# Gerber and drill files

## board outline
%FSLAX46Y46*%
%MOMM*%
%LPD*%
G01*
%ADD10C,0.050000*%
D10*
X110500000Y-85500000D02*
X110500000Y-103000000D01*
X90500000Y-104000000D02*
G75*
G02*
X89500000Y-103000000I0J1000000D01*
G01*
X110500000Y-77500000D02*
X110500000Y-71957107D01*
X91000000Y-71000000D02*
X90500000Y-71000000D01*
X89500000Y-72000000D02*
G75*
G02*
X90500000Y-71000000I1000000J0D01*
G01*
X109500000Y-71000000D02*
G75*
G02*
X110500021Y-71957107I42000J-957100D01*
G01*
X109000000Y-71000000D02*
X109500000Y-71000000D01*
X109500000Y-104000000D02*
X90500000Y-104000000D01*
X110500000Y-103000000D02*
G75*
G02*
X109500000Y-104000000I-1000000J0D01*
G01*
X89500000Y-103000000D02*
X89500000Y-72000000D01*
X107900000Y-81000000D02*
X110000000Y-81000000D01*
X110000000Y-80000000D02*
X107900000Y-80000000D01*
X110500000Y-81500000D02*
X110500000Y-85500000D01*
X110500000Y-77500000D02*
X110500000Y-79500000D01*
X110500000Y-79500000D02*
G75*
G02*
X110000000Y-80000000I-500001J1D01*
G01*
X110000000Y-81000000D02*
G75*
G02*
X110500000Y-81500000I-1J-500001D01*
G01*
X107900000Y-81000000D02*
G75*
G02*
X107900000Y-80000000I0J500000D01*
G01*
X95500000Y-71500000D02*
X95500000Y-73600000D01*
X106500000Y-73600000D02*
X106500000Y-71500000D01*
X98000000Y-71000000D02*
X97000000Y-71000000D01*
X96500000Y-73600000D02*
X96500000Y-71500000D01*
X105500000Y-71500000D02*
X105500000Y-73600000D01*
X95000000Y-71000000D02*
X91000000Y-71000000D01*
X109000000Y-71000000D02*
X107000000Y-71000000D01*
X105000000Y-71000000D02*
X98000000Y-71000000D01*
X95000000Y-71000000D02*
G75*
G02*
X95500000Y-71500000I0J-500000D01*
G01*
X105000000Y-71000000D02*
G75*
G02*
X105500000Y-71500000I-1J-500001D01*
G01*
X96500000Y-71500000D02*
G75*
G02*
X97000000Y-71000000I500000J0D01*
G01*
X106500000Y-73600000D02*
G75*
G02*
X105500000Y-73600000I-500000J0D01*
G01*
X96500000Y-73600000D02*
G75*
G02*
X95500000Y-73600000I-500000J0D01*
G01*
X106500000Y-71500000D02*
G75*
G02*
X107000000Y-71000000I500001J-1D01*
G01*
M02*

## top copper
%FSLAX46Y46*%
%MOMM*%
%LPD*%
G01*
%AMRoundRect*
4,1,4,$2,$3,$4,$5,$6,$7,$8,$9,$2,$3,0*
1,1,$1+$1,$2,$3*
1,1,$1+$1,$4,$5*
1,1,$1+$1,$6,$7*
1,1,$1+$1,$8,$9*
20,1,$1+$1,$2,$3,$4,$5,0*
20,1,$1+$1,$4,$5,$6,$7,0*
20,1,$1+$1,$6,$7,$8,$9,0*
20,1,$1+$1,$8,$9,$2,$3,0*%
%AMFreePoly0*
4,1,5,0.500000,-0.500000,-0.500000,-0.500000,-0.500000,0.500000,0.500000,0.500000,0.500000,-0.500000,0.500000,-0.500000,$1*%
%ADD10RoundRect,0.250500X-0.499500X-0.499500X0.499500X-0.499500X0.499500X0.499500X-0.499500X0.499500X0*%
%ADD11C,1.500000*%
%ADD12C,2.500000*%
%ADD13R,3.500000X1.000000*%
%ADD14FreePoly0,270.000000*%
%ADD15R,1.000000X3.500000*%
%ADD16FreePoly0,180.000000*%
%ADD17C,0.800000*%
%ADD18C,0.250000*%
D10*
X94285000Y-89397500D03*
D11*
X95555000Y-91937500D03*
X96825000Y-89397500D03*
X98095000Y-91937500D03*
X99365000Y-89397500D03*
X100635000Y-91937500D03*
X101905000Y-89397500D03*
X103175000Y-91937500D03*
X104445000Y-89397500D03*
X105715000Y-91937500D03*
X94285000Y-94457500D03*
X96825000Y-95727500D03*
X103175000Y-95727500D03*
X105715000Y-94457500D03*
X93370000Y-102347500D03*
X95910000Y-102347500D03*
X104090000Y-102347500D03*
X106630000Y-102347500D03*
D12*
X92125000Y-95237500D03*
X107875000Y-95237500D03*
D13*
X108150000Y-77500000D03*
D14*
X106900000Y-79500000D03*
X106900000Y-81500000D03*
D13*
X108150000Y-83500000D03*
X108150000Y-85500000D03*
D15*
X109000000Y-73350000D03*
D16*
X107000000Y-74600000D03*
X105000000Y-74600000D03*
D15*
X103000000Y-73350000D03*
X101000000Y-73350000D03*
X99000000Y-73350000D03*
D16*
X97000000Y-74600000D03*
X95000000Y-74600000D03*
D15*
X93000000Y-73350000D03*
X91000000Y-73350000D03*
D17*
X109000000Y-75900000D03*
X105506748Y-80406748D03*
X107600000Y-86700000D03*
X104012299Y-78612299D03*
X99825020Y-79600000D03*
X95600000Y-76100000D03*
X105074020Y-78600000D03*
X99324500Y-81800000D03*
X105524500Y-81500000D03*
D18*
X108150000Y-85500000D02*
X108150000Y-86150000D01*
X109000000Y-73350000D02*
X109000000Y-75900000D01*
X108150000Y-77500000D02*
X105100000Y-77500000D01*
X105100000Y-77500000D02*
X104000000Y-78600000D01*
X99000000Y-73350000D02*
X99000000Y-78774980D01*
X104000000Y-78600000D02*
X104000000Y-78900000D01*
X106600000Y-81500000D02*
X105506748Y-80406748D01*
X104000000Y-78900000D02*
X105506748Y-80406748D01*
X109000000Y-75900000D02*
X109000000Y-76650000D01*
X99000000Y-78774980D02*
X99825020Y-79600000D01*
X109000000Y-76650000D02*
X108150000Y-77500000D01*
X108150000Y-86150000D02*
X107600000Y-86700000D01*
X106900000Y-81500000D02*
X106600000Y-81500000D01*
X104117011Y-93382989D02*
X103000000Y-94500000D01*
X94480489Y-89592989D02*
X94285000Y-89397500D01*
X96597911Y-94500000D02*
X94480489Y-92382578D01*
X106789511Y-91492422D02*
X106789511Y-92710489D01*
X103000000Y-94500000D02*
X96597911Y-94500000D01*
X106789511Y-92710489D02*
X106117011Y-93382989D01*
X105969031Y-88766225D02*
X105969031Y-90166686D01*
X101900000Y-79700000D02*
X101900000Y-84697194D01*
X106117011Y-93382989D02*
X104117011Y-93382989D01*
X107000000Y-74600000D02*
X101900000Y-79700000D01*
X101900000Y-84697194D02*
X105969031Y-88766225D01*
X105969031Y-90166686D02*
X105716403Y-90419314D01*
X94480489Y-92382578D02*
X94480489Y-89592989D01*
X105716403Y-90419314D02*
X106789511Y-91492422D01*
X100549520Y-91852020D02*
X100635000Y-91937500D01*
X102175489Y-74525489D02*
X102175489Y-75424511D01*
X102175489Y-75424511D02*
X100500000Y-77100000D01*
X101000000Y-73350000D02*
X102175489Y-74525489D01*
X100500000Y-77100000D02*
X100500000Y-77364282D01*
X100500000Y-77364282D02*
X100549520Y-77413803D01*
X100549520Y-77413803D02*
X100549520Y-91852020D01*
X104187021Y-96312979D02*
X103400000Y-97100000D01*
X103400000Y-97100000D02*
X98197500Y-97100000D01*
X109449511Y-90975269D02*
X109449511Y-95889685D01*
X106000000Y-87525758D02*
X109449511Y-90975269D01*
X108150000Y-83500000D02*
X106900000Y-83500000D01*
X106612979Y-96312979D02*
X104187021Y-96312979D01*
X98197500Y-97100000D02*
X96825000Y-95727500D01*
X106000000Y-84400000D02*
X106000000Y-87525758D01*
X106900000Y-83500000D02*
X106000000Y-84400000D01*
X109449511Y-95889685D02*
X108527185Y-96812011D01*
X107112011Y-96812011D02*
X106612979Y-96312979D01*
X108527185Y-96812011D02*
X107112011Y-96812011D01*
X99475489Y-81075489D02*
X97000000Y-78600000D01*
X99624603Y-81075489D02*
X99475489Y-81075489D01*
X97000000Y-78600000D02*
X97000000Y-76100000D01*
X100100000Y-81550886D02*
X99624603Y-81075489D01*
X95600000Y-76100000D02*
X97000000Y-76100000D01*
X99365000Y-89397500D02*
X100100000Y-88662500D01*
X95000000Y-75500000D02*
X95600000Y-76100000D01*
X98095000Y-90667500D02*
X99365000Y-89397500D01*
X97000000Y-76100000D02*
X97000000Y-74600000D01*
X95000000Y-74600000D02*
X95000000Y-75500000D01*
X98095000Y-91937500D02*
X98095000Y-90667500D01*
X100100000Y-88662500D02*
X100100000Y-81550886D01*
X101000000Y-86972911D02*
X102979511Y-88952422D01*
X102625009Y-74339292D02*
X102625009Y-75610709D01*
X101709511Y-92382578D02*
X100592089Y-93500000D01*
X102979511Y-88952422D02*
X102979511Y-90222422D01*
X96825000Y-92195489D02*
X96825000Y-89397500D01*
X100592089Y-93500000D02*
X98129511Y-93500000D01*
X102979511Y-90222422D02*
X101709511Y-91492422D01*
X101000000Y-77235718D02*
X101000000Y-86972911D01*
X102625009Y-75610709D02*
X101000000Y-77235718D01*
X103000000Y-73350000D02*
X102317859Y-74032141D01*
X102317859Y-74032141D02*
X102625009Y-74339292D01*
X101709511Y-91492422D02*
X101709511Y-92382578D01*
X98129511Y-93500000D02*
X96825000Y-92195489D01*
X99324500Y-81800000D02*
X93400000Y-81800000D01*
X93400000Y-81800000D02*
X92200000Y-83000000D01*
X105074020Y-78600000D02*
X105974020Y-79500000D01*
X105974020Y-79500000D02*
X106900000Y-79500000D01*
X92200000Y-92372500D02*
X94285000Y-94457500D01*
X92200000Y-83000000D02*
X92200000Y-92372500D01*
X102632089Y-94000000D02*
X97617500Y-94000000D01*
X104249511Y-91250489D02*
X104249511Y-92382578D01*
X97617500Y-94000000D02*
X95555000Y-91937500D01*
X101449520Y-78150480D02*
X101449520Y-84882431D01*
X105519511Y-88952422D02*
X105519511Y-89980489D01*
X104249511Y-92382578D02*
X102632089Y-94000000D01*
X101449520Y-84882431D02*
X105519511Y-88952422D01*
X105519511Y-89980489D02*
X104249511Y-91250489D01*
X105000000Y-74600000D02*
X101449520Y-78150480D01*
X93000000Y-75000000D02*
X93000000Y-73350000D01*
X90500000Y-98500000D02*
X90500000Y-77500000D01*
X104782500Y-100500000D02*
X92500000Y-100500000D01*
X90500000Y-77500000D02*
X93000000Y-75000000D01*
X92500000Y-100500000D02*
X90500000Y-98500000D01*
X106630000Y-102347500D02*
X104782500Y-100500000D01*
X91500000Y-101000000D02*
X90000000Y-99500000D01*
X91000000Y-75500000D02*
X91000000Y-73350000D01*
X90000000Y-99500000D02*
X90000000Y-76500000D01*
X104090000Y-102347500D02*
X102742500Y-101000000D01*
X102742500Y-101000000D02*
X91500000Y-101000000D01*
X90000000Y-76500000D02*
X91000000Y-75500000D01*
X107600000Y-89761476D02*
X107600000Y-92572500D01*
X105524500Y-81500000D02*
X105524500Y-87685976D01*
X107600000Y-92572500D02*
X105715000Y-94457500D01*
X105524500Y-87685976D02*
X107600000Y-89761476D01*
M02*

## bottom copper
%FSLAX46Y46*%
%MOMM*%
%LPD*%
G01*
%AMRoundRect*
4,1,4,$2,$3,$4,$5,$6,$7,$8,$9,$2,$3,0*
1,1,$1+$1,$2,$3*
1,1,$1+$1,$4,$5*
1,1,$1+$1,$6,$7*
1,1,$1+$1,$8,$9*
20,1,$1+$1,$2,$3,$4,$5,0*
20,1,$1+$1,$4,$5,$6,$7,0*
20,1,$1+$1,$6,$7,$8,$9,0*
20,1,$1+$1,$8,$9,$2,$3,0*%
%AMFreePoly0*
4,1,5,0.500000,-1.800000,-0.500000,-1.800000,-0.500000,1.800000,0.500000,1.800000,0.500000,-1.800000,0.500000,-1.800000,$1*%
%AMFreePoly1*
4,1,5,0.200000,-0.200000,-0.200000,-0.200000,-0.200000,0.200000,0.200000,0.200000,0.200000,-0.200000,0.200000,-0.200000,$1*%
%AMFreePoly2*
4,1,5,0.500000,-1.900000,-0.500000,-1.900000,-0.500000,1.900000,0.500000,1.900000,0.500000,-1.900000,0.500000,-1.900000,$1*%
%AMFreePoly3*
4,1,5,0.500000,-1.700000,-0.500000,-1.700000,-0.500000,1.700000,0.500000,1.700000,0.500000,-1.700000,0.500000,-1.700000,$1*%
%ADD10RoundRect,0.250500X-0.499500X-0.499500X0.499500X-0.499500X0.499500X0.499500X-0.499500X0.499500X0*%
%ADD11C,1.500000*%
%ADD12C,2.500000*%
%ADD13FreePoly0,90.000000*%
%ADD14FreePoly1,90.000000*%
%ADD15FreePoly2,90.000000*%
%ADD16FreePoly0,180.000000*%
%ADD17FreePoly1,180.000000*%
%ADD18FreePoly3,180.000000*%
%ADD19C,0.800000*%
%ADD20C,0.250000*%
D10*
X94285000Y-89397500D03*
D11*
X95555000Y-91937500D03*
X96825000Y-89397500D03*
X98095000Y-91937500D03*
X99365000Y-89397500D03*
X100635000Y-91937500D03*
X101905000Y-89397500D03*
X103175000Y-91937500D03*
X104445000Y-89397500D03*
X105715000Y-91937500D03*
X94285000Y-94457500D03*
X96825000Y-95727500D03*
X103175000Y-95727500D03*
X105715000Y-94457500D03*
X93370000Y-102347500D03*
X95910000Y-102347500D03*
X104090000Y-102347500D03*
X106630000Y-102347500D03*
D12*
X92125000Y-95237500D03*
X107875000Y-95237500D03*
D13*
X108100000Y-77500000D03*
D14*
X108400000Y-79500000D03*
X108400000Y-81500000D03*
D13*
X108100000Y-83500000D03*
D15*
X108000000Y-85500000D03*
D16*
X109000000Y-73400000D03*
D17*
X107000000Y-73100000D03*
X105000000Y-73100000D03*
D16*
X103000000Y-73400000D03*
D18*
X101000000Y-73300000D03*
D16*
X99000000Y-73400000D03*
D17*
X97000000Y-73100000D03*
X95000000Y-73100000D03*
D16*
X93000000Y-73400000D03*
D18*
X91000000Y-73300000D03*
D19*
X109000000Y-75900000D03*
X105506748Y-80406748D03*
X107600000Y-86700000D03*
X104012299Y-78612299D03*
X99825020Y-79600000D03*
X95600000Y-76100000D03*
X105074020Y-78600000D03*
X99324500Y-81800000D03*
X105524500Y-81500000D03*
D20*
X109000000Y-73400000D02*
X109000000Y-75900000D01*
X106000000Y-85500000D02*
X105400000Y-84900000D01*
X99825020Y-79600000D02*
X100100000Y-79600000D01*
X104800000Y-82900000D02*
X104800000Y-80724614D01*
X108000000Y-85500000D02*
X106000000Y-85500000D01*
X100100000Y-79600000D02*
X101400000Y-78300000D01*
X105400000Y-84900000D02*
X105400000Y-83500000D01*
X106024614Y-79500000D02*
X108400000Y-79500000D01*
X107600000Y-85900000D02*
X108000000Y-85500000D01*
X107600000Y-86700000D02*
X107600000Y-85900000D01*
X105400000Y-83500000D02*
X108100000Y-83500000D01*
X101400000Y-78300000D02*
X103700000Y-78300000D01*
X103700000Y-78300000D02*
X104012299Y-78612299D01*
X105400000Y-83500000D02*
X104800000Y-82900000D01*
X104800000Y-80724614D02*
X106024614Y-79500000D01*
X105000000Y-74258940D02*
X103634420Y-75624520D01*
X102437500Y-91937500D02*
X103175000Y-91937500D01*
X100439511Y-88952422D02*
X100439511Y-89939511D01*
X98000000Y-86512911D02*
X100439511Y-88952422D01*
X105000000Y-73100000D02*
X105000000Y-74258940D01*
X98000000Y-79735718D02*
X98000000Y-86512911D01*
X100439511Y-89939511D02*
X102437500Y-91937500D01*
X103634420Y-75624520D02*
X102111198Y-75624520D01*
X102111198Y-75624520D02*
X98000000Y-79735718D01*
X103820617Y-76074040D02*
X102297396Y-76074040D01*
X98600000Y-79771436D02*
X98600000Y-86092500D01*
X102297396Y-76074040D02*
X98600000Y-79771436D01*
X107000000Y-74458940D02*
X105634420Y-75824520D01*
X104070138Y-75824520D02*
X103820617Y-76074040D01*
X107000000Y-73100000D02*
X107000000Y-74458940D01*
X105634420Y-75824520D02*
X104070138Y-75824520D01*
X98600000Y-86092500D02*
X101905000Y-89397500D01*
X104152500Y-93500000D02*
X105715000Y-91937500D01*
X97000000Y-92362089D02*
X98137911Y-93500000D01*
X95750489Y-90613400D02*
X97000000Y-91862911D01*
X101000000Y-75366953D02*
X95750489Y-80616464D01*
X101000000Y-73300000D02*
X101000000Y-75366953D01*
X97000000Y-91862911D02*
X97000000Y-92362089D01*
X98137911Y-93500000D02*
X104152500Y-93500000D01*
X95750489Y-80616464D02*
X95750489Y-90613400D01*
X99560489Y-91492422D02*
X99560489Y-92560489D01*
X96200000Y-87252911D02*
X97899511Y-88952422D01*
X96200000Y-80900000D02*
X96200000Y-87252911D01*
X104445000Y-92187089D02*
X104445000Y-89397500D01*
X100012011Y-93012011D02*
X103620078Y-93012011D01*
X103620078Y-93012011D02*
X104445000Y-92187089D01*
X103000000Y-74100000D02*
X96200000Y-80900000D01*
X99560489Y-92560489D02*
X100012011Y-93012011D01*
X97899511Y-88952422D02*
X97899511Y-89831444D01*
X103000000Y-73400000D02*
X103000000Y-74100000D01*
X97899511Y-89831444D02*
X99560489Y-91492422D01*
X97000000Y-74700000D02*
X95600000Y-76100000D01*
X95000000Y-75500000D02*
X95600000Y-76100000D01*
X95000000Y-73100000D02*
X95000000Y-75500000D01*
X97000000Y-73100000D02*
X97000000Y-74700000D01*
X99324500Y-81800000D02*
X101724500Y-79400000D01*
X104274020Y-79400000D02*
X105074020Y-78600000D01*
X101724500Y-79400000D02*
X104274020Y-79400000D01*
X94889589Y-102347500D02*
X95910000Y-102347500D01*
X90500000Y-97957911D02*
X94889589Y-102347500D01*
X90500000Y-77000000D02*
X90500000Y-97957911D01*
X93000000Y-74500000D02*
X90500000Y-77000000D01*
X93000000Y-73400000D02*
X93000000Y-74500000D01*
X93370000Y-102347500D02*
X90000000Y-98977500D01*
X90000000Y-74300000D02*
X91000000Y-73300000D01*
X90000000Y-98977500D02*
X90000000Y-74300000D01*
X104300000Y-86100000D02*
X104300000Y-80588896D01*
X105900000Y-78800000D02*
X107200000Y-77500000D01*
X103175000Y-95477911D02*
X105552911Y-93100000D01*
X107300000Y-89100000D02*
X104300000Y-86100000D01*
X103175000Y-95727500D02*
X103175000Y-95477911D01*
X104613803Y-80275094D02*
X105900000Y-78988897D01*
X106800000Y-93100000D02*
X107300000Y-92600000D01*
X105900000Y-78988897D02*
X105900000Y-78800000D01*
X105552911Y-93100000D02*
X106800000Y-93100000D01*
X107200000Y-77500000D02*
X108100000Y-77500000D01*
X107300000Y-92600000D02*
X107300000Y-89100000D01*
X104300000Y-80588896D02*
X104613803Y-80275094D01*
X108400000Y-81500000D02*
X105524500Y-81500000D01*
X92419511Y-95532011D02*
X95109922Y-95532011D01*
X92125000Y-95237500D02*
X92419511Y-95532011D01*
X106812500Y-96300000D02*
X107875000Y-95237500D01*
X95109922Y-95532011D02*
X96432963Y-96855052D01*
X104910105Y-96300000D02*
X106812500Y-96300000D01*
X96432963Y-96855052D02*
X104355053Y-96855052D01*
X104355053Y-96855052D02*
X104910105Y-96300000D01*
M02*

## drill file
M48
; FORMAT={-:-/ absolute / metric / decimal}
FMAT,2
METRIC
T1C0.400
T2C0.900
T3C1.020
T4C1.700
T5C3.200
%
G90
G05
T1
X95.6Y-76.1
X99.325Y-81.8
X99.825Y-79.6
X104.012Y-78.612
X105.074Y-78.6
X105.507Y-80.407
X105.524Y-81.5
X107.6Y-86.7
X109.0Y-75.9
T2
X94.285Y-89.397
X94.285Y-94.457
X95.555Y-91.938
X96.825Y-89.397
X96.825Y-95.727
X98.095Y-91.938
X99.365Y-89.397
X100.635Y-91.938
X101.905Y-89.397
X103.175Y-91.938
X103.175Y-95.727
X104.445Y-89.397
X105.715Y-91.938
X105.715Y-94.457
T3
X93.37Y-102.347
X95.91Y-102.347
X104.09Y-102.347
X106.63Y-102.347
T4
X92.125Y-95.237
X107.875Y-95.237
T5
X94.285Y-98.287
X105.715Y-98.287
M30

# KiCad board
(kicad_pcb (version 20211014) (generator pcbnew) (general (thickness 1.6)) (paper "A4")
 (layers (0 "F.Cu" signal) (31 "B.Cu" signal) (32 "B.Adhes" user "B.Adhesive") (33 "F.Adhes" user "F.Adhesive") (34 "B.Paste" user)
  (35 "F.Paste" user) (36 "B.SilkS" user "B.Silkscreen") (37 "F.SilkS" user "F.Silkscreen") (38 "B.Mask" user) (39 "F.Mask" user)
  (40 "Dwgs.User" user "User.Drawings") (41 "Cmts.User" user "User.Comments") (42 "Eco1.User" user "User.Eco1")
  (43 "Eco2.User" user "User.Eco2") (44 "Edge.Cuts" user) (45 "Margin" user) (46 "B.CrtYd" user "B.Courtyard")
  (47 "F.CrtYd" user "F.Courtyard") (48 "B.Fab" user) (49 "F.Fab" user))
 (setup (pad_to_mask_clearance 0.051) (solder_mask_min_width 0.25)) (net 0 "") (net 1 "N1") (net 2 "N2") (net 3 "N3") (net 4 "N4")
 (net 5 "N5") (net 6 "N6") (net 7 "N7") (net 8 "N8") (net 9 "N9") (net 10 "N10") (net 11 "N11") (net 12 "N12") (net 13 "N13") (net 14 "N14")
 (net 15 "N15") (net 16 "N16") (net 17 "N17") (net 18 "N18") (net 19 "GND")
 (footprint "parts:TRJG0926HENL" (layer "F.Cu") (at 100 98.2875)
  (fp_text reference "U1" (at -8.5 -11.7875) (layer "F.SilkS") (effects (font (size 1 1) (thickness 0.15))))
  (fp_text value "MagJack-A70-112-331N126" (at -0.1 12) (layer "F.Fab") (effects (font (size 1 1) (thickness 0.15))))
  (pad "" np_thru_hole circle locked (at -5.715 0) (size 3.2 3.2) (drill 3.2) (layers *.Cu *.Mask))
  (pad "" np_thru_hole circle locked (at 5.715 0) (size 3.2 3.2) (drill 3.2) (layers *.Cu *.Mask))
  (pad "1" thru_hole roundrect locked (at -5.715 -8.89) (size 1.5 1.5) (drill 0.9) (layers *.Cu *.Mask) (roundrect_rratio 0.167)
   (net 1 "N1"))
  (pad "2" thru_hole circle locked (at -4.445 -6.35) (size 1.5 1.5) (drill 0.9) (layers *.Cu *.Mask) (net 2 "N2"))
  (pad "3" thru_hole circle locked (at -3.175 -8.89) (size 1.5 1.5) (drill 0.9) (layers *.Cu *.Mask) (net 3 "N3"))
  (pad "4" thru_hole circle locked (at -1.905 -6.35) (size 1.5 1.5) (drill 0.9) (layers *.Cu *.Mask) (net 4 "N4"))
  (pad "5" thru_hole circle locked (at -0.635 -8.89) (size 1.5 1.5) (drill 0.9) (layers *.Cu *.Mask) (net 4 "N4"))
  (pad "6" thru_hole circle locked (at 0.635 -6.35 90) (size 1.5 1.5) (drill 0.9) (layers *.Cu *.Mask) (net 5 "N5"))
  (pad "7" thru_hole circle locked (at 1.905 -8.89) (size 1.5 1.5) (drill 0.9) (layers *.Cu *.Mask) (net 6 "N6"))
  (pad "8" thru_hole circle locked (at 3.175 -6.35) (size 1.5 1.5) (drill 0.9) (layers *.Cu *.Mask) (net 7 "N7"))
  (pad "9" thru_hole circle locked (at 4.445 -8.89) (size 1.5 1.5) (drill 0.9) (layers *.Cu *.Mask) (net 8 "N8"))
  (pad "10" thru_hole circle locked (at 5.715 -6.35) (size 1.5 1.5) (drill 0.9) (layers *.Cu *.Mask) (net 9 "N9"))
  (pad "11" thru_hole circle locked (at -5.715 -3.83) (size 1.5 1.5) (drill 0.9) (layers *.Cu *.Mask) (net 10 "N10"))
  (pad "12" thru_hole circle locked (at -3.175 -2.56) (size 1.5 1.5) (drill 0.9) (layers *.Cu *.Mask) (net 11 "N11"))
  (pad "13" thru_hole circle locked (at 3.175 -2.56) (size 1.5 1.5) (drill 0.9) (layers *.Cu *.Mask) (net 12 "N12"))
  (pad "14" thru_hole circle locked (at 5.715 -3.83) (size 1.5 1.5) (drill 0.9) (layers *.Cu *.Mask) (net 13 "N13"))
  (pad "15" thru_hole circle locked (at -6.63 4.06) (size 1.5 1.5) (drill 1.02) (layers *.Cu *.Mask) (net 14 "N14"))
  (pad "16" thru_hole circle locked (at -4.09 4.06) (size 1.5 1.5) (drill 1.02) (layers *.Cu *.Mask) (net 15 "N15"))
  (pad "17" thru_hole circle locked (at 4.09 4.06) (size 1.5 1.5) (drill 1.02) (layers *.Cu *.Mask) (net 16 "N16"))
  (pad "18" thru_hole circle locked (at 6.63 4.06) (size 1.5 1.5) (drill 1.02) (layers *.Cu *.Mask) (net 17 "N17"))
  (pad "19" thru_hole circle locked (at -7.875 -3.05) (size 2.5 2.5) (drill 1.7) (layers *.Cu *.Mask) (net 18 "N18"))
  (pad "20" thru_hole circle locked (at 7.875 -3.05) (size 2.5 2.5) (drill 1.7) (layers *.Cu *.Mask) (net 18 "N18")))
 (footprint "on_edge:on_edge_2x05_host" (layer "F.Cu") (at 110.5 81.5 -90)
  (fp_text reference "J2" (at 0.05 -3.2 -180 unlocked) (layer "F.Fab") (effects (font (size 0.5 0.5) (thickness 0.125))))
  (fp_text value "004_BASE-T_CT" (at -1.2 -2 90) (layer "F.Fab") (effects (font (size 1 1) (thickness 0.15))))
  (fp_line (start -0.5 2.6) (end -0.5 0.5) (layer "Edge.Cuts") (width 0.05))
  (fp_line (start -1.5 0.5) (end -1.5 2.6) (layer "Edge.Cuts") (width 0.05))
  (fp_line (start 0 0) (end 4 0) (layer "Edge.Cuts") (width 0.05))
  (fp_line (start -4 0) (end -2 0) (layer "Edge.Cuts") (width 0.05))
  (fp_arc (start -2 0) (mid -1.646447 0.146447) (end -1.5 0.5) (layer "Edge.Cuts") (width 0.05))
  (fp_arc (start -0.5 0.5) (mid -0.353553 0.146447) (end 0 0) (layer "Edge.Cuts") (width 0.05))
  (fp_arc (start -0.5 2.6) (mid -1 3.1) (end -1.5 2.6) (layer "Edge.Cuts") (width 0.05))
  (pad "1" smd rect locked (at -4 2.35 270) (size 1 3.5) (layers "F.Cu" "F.Mask") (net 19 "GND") (zone_connect 0))
  (pad "2" smd custom locked (at -2 3.6 270) (size 1 1) (layers "F.Cu" "F.Mask") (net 10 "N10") (zone_connect 0)
   (options (clearance outline) (anchor rect)) (primitives))
  (pad "3" smd custom locked (at 0 3.6 270) (size 1 1) (layers "F.Cu" "F.Mask") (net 19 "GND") (zone_connect 0)
   (options (clearance outline) (anchor rect)) (primitives))
  (pad "4" smd rect locked (at 2 2.35 270) (size 1 3.5) (layers "F.Cu" "F.Mask") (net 11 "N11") (zone_connect 0))
  (pad "5" smd rect locked (at 4 2.35 270) (size 1 3.5) (layers "F.Cu" "F.Mask") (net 19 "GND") (zone_connect 0))
  (pad "6" smd custom locked (at -4 2.4 90) (size 1 3.6) (layers "B.Cu" "B.Mask") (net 12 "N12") (zone_connect 0)
   (options (clearance outline) (anchor rect)) (primitives))
  (pad "7" smd custom locked (at -2 2.1 90) (size 0.4 0.4) (layers "B.Cu" "B.Mask") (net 19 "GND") (zone_connect 0)
   (options (clearance outline) (anchor rect)) (primitives))
  (pad "8" smd custom locked (at 0 2.1 90) (size 0.4 0.4) (layers "B.Cu" "B.Mask") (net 13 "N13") (zone_connect 0)
   (options (clearance outline) (anchor rect)) (primitives))
  (pad "9" smd custom locked (at 2 2.4 90) (size 1 3.6) (layers "B.Cu" "B.Mask") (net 19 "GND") (zone_connect 0)
   (options (clearance outline) (anchor rect)) (primitives))
  (pad "10" smd custom locked (at 4 2.5 90) (size 1 3.8) (layers "B.Cu" "B.Mask") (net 19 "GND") (zone_connect 0)
   (options (clearance outline) (anchor rect)) (primitives)))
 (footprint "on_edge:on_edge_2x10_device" (layer "F.Cu") (at 105 71 180)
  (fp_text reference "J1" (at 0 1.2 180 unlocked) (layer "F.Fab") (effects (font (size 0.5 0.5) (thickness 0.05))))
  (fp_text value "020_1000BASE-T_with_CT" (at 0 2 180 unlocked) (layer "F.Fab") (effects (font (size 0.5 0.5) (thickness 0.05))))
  (fp_line (start 9.5 -0.5) (end 9.5 -2.6) (layer "Edge.Cuts") (width 0.05))
  (fp_line (start -1.5 -2.6) (end -1.5 -0.5) (layer "Edge.Cuts") (width 0.05))
  (fp_line (start 7 0) (end 8 0) (layer "Edge.Cuts") (width 0.05))
  (fp_line (start 8.5 -2.6) (end 8.5 -0.5) (layer "Edge.Cuts") (width 0.05))
  (fp_line (start -0.5 -0.5) (end -0.5 -2.6) (layer "Edge.Cuts") (width 0.05))
  (fp_line (start 10 0) (end 14 0) (layer "Edge.Cuts") (width 0.05))
  (fp_line (start -4 0) (end -2 0) (layer "Edge.Cuts") (width 0.05))
  (fp_line (start 0 0) (end 7 0) (layer "Edge.Cuts") (width 0.05))
  (fp_arc (start 10 0) (mid 9.646447 -0.146447) (end 9.5 -0.5) (layer "Edge.Cuts") (width 0.05))
  (fp_arc (start 0 0) (mid -0.353553 -0.146447) (end -0.5 -0.5) (layer "Edge.Cuts") (width 0.05))
  (fp_arc (start 8.5 -0.5) (mid 8.353553 -0.146447) (end 8 0) (layer "Edge.Cuts") (width 0.05))
  (fp_arc (start -1.5 -2.6) (mid -1 -3.1) (end -0.5 -2.6) (layer "Edge.Cuts") (width 0.05))
  (fp_arc (start 8.5 -2.6) (mid 9 -3.1) (end 9.5 -2.6) (layer "Edge.Cuts") (width 0.05))
  (fp_arc (start -1.5 -0.5) (mid -1.646447 -0.146447) (end -2 0) (layer "Edge.Cuts") (width 0.05))
  (pad "1" smd rect locked (at -4 -2.35) (size 1 3.5) (layers "F.Cu" "F.Mask") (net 19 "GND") (zone_connect 0))
  (pad "2" smd custom locked (at -2 -3.6 180) (size 1 1) (layers "F.Cu" "F.Mask") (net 1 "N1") (zone_connect 0)
   (options (clearance outline) (anchor rect)) (primitives))
  (pad "3" smd custom locked (at 0 -3.6 180) (size 1 1) (layers "F.Cu" "F.Mask") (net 2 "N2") (zone_connect 0)
   (options (clearance outline) (anchor rect)) (primitives))
  (pad "4" smd rect locked (at 2 -2.35) (size 1 3.5) (layers "F.Cu" "F.Mask") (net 3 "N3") (zone_connect 0))
  (pad "5" smd rect locked (at 4 -2.35) (size 1 3.5) (layers "F.Cu" "F.Mask") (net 5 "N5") (zone_connect 0))
  (pad "6" smd rect locked (at 6 -2.35) (size 1 3.5) (layers "F.Cu" "F.Mask") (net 19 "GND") (zone_connect 0))
  (pad "7" smd custom locked (at 8 -3.6 180) (size 1 1) (layers "F.Cu" "F.Mask") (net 4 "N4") (zone_connect 0)
   (options (clearance outline) (anchor rect)) (primitives))
  (pad "8" smd custom locked (at 10 -3.6 180) (size 1 1) (layers "F.Cu" "F.Mask") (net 4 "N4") (zone_connect 0)
   (options (clearance outline) (anchor rect)) (primitives))
  (pad "9" smd rect locked (at 12 -2.35) (size 1 3.5) (layers "F.Cu" "F.Mask") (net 17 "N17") (zone_connect 0))
  (pad "10" smd rect locked (at 14 -2.35) (size 1 3.5) (layers "F.Cu" "F.Mask") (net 16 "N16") (zone_connect 0))
  (pad "11" smd custom locked (at -4 -2.4 180) (size 1 3.6) (layers "B.Cu" "B.Mask") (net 19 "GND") (zone_connect 0)
   (options (clearance outline) (anchor rect)) (primitives))
  (pad "12" smd custom locked (at -2 -2.1 180) (size 0.4 0.4) (layers "B.Cu" "B.Mask") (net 6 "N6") (zone_connect 0)
   (options (clearance outline) (anchor rect)) (primitives))
  (pad "13" smd custom locked (at 0 -2.1 180) (size 0.4 0.4) (layers "B.Cu" "B.Mask") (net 7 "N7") (zone_connect 0)
   (options (clearance outline) (anchor rect)) (primitives))
  (pad "14" smd custom locked (at 2 -2.4 180) (size 1 3.6) (layers "B.Cu" "B.Mask") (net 8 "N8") (zone_connect 0)
   (options (clearance outline) (anchor rect)) (primitives))
  (pad "15" smd custom locked (at 4 -2.3 180) (size 1 3.4) (layers "B.Cu" "B.Mask") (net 9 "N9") (zone_connect 0)
   (options (clearance outline) (anchor rect)) (primitives))
  (pad "16" smd custom locked (at 6 -2.4 180) (size 1 3.6) (layers "B.Cu" "B.Mask") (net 19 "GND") (zone_connect 0)
   (options (clearance outline) (anchor rect)) (primitives))
  (pad "17" smd custom locked (at 8 -2.1 180) (size 0.4 0.4) (layers "B.Cu" "B.Mask") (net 4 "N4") (zone_connect 0)
   (options (clearance outline) (anchor rect)) (primitives))
  (pad "18" smd custom locked (at 10 -2.1 180) (size 0.4 0.4) (layers "B.Cu" "B.Mask") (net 4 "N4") (zone_connect 0)
   (options (clearance outline) (anchor rect)) (primitives))
  (pad "19" smd custom locked (at 12 -2.4 180) (size 1 3.6) (layers "B.Cu" "B.Mask") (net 15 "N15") (zone_connect 0)
   (options (clearance outline) (anchor rect)) (primitives))
  (pad "20" smd custom locked (at 14 -2.3 180) (size 1 3.4) (layers "B.Cu" "B.Mask") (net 14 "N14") (zone_connect 0)
   (options (clearance outline) (anchor rect)) (primitives)))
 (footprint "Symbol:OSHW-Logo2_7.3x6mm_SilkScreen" (layer "B.Cu") (at 99 82 180)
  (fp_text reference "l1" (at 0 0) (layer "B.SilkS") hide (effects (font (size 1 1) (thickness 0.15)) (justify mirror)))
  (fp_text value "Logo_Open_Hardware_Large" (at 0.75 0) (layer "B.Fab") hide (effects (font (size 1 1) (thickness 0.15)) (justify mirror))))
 (gr_line (start 110.5 85.5) (end 110.5 103) (layer "Edge.Cuts") (width 0.05))
 (gr_arc (start 90.5 104) (mid 89.792893 103.707107) (end 89.5 103) (layer "Edge.Cuts") (width 0.05))
 (gr_line (start 110.5 77.5) (end 110.5 71.957107) (layer "Edge.Cuts") (width 0.05))
 (gr_line (start 91 71) (end 90.5 71) (layer "Edge.Cuts") (width 0.05))
 (gr_arc (start 89.5 72) (mid 89.792893 71.292893) (end 90.5 71) (layer "Edge.Cuts") (width 0.05))
 (gr_arc (start 109.5 71) (mid 110.204395 71.264999) (end 110.5 71.957107) (layer "Edge.Cuts") (width 0.05))
 (gr_line (start 109 71) (end 109.5 71) (layer "Edge.Cuts") (width 0.05))
 (gr_line (start 109.5 104) (end 90.5 104) (layer "Edge.Cuts") (width 0.05))
 (gr_arc (start 110.5 103) (mid 110.207107 103.707107) (end 109.5 104) (layer "Edge.Cuts") (width 0.05))
 (gr_line (start 89.5 103) (end 89.5 72) (layer "Edge.Cuts") (width 0.05))
 (segment (start 108.15 85.5) (end 108.15 86.15) (width 0.25) (layer "F.Cu") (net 19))
 (segment (start 109 73.35) (end 109 75.9) (width 0.25) (layer "F.Cu") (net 19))
 (segment (start 108.15 77.5) (end 105.1 77.5) (width 0.25) (layer "F.Cu") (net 19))
 (segment (start 105.1 77.5) (end 104 78.6) (width 0.25) (layer "F.Cu") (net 19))
 (segment (start 99 73.35) (end 99 78.77498) (width 0.25) (layer "F.Cu") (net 19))
 (segment (start 104 78.6) (end 104 78.9) (width 0.25) (layer "F.Cu") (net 19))
 (segment (start 106.6 81.5) (end 105.506748 80.406748) (width 0.25) (layer "F.Cu") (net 19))
 (segment (start 104 78.9) (end 105.506748 80.406748) (width 0.25) (layer "F.Cu") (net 19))
 (segment (start 109 75.9) (end 109 76.65) (width 0.25) (layer "F.Cu") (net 19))
 (segment (start 99 78.77498) (end 99.82502 79.6) (width 0.25) (layer "F.Cu") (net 19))
 (segment (start 109 76.65) (end 108.15 77.5) (width 0.25) (layer "F.Cu") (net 19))
 (segment (start 108.15 86.15) (end 107.6 86.7) (width 0.25) (layer "F.Cu") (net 19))
 (segment (start 106.9 81.5) (end 106.6 81.5) (width 0.25) (layer "F.Cu") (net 19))
 (via (at 109 75.9) (size 0.8) (drill 0.4) (layers "F.Cu" "B.Cu") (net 19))
 (via (at 105.506748 80.406748) (size 0.8) (drill 0.4) (layers "F.Cu" "B.Cu") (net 19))
 (via (at 107.6 86.7) (size 0.8) (drill 0.4) (layers "F.Cu" "B.Cu") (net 19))
 (via (at 104.012299 78.612299) (size 0.8) (drill 0.4) (layers "F.Cu" "B.Cu") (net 19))
 (via (at 99.82502 79.6) (size 0.8) (drill 0.4) (layers "F.Cu" "B.Cu") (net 19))
 (segment (start 109 73.4) (end 109 75.9) (width 0.25) (layer "B.Cu") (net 19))
 (segment (start 106 85.5) (end 105.4 84.9) (width 0.25) (layer "B.Cu") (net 19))
 (segment (start 99.82502 79.6) (end 100.1 79.6) (width 0.25) (layer "B.Cu") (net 19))
 (segment (start 104.8 82.9) (end 104.8 80.724614) (width 0.25) (layer "B.Cu") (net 19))
 (segment (start 108 85.5) (end 106 85.5) (width 0.25) (layer "B.Cu") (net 19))
 (segment (start 100.1 79.6) (end 101.4 78.3) (width 0.25) (layer "B.Cu") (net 19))
 (segment (start 105.4 84.9) (end 105.4 83.5) (width 0.25) (layer "B.Cu") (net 19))
 (segment (start 106.024614 79.5) (end 108.4 79.5) (width 0.25) (layer "B.Cu") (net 19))
 (segment (start 107.6 85.9) (end 108 85.5) (width 0.25) (layer "B.Cu") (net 19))
 (segment (start 107.6 86.7) (end 107.6 85.9) (width 0.25) (layer "B.Cu") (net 19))
 (segment (start 105.4 83.5) (end 108.1 83.5) (width 0.25) (layer "B.Cu") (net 19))
 (segment (start 101.4 78.3) (end 103.7 78.3) (width 0.25) (layer "B.Cu") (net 19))
 (segment (start 103.7 78.3) (end 104.012299 78.612299) (width 0.25) (layer "B.Cu") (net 19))
 (segment (start 105.4 83.5) (end 104.8 82.9) (width 0.25) (layer "B.Cu") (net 19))
 (segment (start 104.8 80.724614) (end 106.024614 79.5) (width 0.25) (layer "B.Cu") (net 19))
 (segment (start 104.117011 93.382989) (end 103 94.5) (width 0.25) (layer "F.Cu") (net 1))
 (segment (start 94.480489 89.592989) (end 94.285 89.3975) (width 0.25) (layer "F.Cu") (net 1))
 (segment (start 96.597911 94.5) (end 94.480489 92.382578) (width 0.25) (layer "F.Cu") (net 1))
 (segment (start 106.789511 91.492422) (end 106.789511 92.710489) (width 0.25) (layer "F.Cu") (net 1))
 (segment (start 103 94.5) (end 96.597911 94.5) (width 0.25) (layer "F.Cu") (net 1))
 (segment (start 106.789511 92.710489) (end 106.117011 93.382989) (width 0.25) (layer "F.Cu") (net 1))
 (segment (start 105.969031 88.766225) (end 105.969031 90.166686) (width 0.25) (layer "F.Cu") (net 1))
 (segment (start 101.9 79.7) (end 101.9 84.697194) (width 0.25) (layer "F.Cu") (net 1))
 (segment (start 106.117011 93.382989) (end 104.117011 93.382989) (width 0.25) (layer "F.Cu") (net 1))
 (segment (start 107 74.6) (end 101.9 79.7) (width 0.25) (layer "F.Cu") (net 1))
 (segment (start 101.9 84.697194) (end 105.969031 88.766225) (width 0.25) (layer "F.Cu") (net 1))
 (segment (start 105.969031 90.166686) (end 105.716403 90.419314) (width 0.25) (layer "F.Cu") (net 1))
 (segment (start 94.480489 92.382578) (end 94.480489 89.592989) (width 0.25) (layer "F.Cu") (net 1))
 (segment (start 105.716403 90.419314) (end 106.789511 91.492422) (width 0.25) (layer "F.Cu") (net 1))
 (segment (start 100.54952 91.85202) (end 100.635 91.9375) (width 0.25) (layer "F.Cu") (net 5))
 (segment (start 102.175489 74.525489) (end 102.175489 75.424511) (width 0.25) (layer "F.Cu") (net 5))
 (segment (start 102.175489 75.424511) (end 100.5 77.1) (width 0.25) (layer "F.Cu") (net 5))
 (segment (start 101 73.35) (end 102.175489 74.525489) (width 0.25) (layer "F.Cu") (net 5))
 (segment (start 100.5 77.1) (end 100.5 77.364282) (width 0.25) (layer "F.Cu") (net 5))
 (segment (start 100.5 77.364282) (end 100.54952 77.413803) (width 0.25) (layer "F.Cu") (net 5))
 (segment (start 100.54952 77.413803) (end 100.54952 91.85202) (width 0.25) (layer "F.Cu") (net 5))
 (segment (start 104.187021 96.312979) (end 103.4 97.1) (width 0.25) (layer "F.Cu") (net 11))
 (segment (start 103.4 97.1) (end 98.1975 97.1) (width 0.25) (layer "F.Cu") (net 11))
 (segment (start 109.449511 90.975269) (end 109.449511 95.889685) (width 0.25) (layer "F.Cu") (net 11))
 (segment (start 106 87.525758) (end 109.449511 90.975269) (width 0.25) (layer "F.Cu") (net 11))
 (segment (start 108.15 83.5) (end 106.9 83.5) (width 0.25) (layer "F.Cu") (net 11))
 (segment (start 106.612979 96.312979) (end 104.187021 96.312979) (width 0.25) (layer "F.Cu") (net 11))
 (segment (start 98.1975 97.1) (end 96.825 95.7275) (width 0.25) (layer "F.Cu") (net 11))
 (segment (start 106 84.4) (end 106 87.525758) (width 0.25) (layer "F.Cu") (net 11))
 (segment (start 106.9 83.5) (end 106 84.4) (width 0.25) (layer "F.Cu") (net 11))
 (segment (start 109.449511 95.889685) (end 108.527185 96.812011) (width 0.25) (layer "F.Cu") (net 11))
 (segment (start 107.112011 96.812011) (end 106.612979 96.312979) (width 0.25) (layer "F.Cu") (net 11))
 (segment (start 108.527185 96.812011) (end 107.112011 96.812011) (width 0.25) (layer "F.Cu") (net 11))
 (segment (start 105 74.25894) (end 103.63442 75.62452) (width 0.25) (layer "B.Cu") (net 7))
 (segment (start 102.4375 91.9375) (end 103.175 91.9375) (width 0.25) (layer "B.Cu") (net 7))
 (segment (start 100.439511 88.952422) (end 100.439511 89.939511) (width 0.25) (layer "B.Cu") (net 7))
 (segment (start 98 86.512911) (end 100.439511 88.952422) (width 0.25) (layer "B.Cu") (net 7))
 (segment (start 105 73.1) (end 105 74.25894) (width 0.25) (layer "B.Cu") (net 7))
 (segment (start 98 79.735718) (end 98 86.512911) (width 0.25) (layer "B.Cu") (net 7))
 (segment (start 100.439511 89.939511) (end 102.4375 91.9375) (width 0.25) (layer "B.Cu") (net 7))
 (segment (start 103.63442 75.62452) (end 102.111198 75.62452) (width 0.25) (layer "B.Cu") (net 7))
 (segment (start 102.111198 75.62452) (end 98 79.735718) (width 0.25) (layer "B.Cu") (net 7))
 (segment (start 103.820617 76.07404) (end 102.297396 76.07404) (width 0.25) (layer "B.Cu") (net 6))
 (segment (start 98.6 79.771436) (end 98.6 86.0925) (width 0.25) (layer "B.Cu") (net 6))
 (segment (start 102.297396 76.07404) (end 98.6 79.771436) (width 0.25) (layer "B.Cu") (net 6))
 (segment (start 107 74.45894) (end 105.63442 75.82452) (width 0.25) (layer "B.Cu") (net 6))
 (segment (start 104.070138 75.82452) (end 103.820617 76.07404) (width 0.25) (layer "B.Cu") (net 6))
 (segment (start 107 73.1) (end 107 74.45894) (width 0.25) (layer "B.Cu") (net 6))
 (segment (start 105.63442 75.82452) (end 104.070138 75.82452) (width 0.25) (layer "B.Cu") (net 6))
 (segment (start 98.6 86.0925) (end 101.905 89.3975) (width 0.25) (layer "B.Cu") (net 6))
 (segment (start 104.1525 93.5) (end 105.715 91.9375) (width 0.25) (layer "B.Cu") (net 9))
 (segment (start 97 92.362089) (end 98.137911 93.5) (width 0.25) (layer "B.Cu") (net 9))
 (segment (start 95.750489 90.6134) (end 97 91.862911) (width 0.25) (layer "B.Cu") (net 9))
 (segment (start 101 75.366953) (end 95.750489 80.616464) (width 0.25) (layer "B.Cu") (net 9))
 (segment (start 101 73.3) (end 101 75.366953) (width 0.25) (layer "B.Cu") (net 9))
 (segment (start 97 91.862911) (end 97 92.362089) (width 0.25) (layer "B.Cu") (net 9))
 (segment (start 98.137911 93.5) (end 104.1525 93.5) (width 0.25) (layer "B.Cu") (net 9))
 (segment (start 95.750489 80.616464) (end 95.750489 90.6134) (width 0.25) (layer "B.Cu") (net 9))
 (segment (start 99.560489 91.492422) (end 99.560489 92.560489) (width 0.25) (layer "B.Cu") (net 8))
 (segment (start 96.2 87.252911) (end 97.899511 88.952422) (width 0.25) (layer "B.Cu") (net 8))
 (segment (start 96.2 80.9) (end 96.2 87.252911) (width 0.25) (layer "B.Cu") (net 8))
 (segment (start 104.445 92.187089) (end 104.445 89.3975) (width 0.25) (layer "B.Cu") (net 8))
 (segment (start 100.012011 93.012011) (end 103.620078 93.012011) (width 0.25) (layer "B.Cu") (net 8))
 (segment (start 103.620078 93.012011) (end 104.445 92.187089) (width 0.25) (layer "B.Cu") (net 8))
 (segment (start 103 74.1) (end 96.2 80.9) (width 0.25) (layer "B.Cu") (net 8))
 (segment (start 99.560489 92.560489) (end 100.012011 93.012011) (width 0.25) (layer "B.Cu") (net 8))
 (segment (start 97.899511 88.952422) (end 97.899511 89.831444) (width 0.25) (layer "B.Cu") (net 8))
 (segment (start 103 73.4) (end 103 74.1) (width 0.25) (layer "B.Cu") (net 8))
 (segment (start 97.899511 89.831444) (end 99.560489 91.492422) (width 0.25) (layer "B.Cu") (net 8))
 (segment (start 99.475489 81.075489) (end 97 78.6) (width 0.25) (layer "F.Cu") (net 4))
 (segment (start 99.624603 81.075489) (end 99.475489 81.075489) (width 0.25) (layer "F.Cu") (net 4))
 (segment (start 97 78.6) (end 97 76.1) (width 0.25) (layer "F.Cu") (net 4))
 (segment (start 100.1 81.550886) (end 99.624603 81.075489) (width 0.25) (layer "F.Cu") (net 4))
 (segment (start 95.6 76.1) (end 97 76.1) (width 0.25) (layer "F.Cu") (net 4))
 (segment (start 99.365 89.3975) (end 100.1 88.6625) (width 0.25) (layer "F.Cu") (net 4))
 (segment (start 95 75.5) (end 95.6 76.1) (width 0.25) (layer "F.Cu") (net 4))
 (segment (start 98.095 90.6675) (end 99.365 89.3975) (width 0.25) (layer "F.Cu") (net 4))
 (segment (start 97 76.1) (end 97 74.6) (width 0.25) (layer "F.Cu") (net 4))
 (segment (start 95 74.6) (end 95 75.5) (width 0.25) (layer "F.Cu") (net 4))
 (segment (start 98.095 91.9375) (end 98.095 90.6675) (width 0.25) (layer "F.Cu") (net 4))
 (segment (start 100.1 88.6625) (end 100.1 81.550886) (width 0.25) (layer "F.Cu") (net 4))
 (via (at 95.6 76.1) (size 0.8) (drill 0.4) (layers "F.Cu" "B.Cu") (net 4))
 (segment (start 97 74.7) (end 95.6 76.1) (width 0.25) (layer "B.Cu") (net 4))
 (segment (start 95 75.5) (end 95.6 76.1) (width 0.25) (layer "B.Cu") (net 4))
 (segment (start 95 73.1) (end 95 75.5) (width 0.25) (layer "B.Cu") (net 4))
 (segment (start 97 73.1) (end 97 74.7) (width 0.25) (layer "B.Cu") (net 4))
 (segment (start 101 86.972911) (end 102.979511 88.952422) (width 0.25) (layer "F.Cu") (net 3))
 (segment (start 102.625009 74.339292) (end 102.625009 75.610709) (width 0.25) (layer "F.Cu") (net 3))
 (segment (start 101.709511 92.382578) (end 100.592089 93.5) (width 0.25) (layer "F.Cu") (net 3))
 (segment (start 102.979511 88.952422) (end 102.979511 90.222422) (width 0.25) (layer "F.Cu") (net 3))
 (segment (start 96.825 92.195489) (end 96.825 89.3975) (width 0.25) (layer "F.Cu") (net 3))
 (segment (start 100.592089 93.5) (end 98.129511 93.5) (width 0.25) (layer "F.Cu") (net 3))
 (segment (start 102.979511 90.222422) (end 101.709511 91.492422) (width 0.25) (layer "F.Cu") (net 3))
 (segment (start 101 77.235718) (end 101 86.972911) (width 0.25) (layer "F.Cu") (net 3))
 (segment (start 102.625009 75.610709) (end 101 77.235718) (width 0.25) (layer "F.Cu") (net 3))
 (segment (start 103 73.35) (end 102.317859 74.032141) (width 0.25) (layer "F.Cu") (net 3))
 (segment (start 102.317859 74.032141) (end 102.625009 74.339292) (width 0.25) (layer "F.Cu") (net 3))
 (segment (start 101.709511 91.492422) (end 101.709511 92.382578) (width 0.25) (layer "F.Cu") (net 3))
 (segment (start 98.129511 93.5) (end 96.825 92.195489) (width 0.25) (layer "F.Cu") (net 3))
 (segment (start 99.3245 81.8) (end 93.4 81.8) (width 0.25) (layer "F.Cu") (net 10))
 (segment (start 93.4 81.8) (end 92.2 83) (width 0.25) (layer "F.Cu") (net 10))
 (segment (start 105.07402 78.6) (end 105.97402 79.5) (width 0.25) (layer "F.Cu") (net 10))
 (segment (start 105.97402 79.5) (end 106.9 79.5) (width 0.25) (layer "F.Cu") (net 10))
 (segment (start 92.2 92.3725) (end 94.285 94.4575) (width 0.25) (layer "F.Cu") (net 10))
 (segment (start 92.2 83) (end 92.2 92.3725) (width 0.25) (layer "F.Cu") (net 10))
 (via (at 105.07402 78.6) (size 0.8) (drill 0.4) (layers "F.Cu" "B.Cu") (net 10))
 (via (at 99.3245 81.8) (size 0.8) (drill 0.4) (layers "F.Cu" "B.Cu") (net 10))
 (segment (start 99.3245 81.8) (end 101.7245 79.4) (width 0.25) (layer "B.Cu") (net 10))
 (segment (start 104.27402 79.4) (end 105.07402 78.6) (width 0.25) (layer "B.Cu") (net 10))
 (segment (start 101.7245 79.4) (end 104.27402 79.4) (width 0.25) (layer "B.Cu") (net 10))
 (segment (start 102.632089 94) (end 97.6175 94) (width 0.25) (layer "F.Cu") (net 2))
 (segment (start 104.249511 91.250489) (end 104.249511 92.382578) (width 0.25) (layer "F.Cu") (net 2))
 (segment (start 97.6175 94) (end 95.555 91.9375) (width 0.25) (layer "F.Cu") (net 2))
 (segment (start 101.44952 78.15048) (end 101.44952 84.882431) (width 0.25) (layer "F.Cu") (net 2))
 (segment (start 105.519511 88.952422) (end 105.519511 89.980489) (width 0.25) (layer "F.Cu") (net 2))
 (segment (start 104.249511 92.382578) (end 102.632089 94) (width 0.25) (layer "F.Cu") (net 2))
 (segment (start 101.44952 84.882431) (end 105.519511 88.952422) (width 0.25) (layer "F.Cu") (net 2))
 (segment (start 105.519511 89.980489) (end 104.249511 91.250489) (width 0.25) (layer "F.Cu") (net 2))
 (segment (start 105 74.6) (end 101.44952 78.15048) (width 0.25) (layer "F.Cu") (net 2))
 (segment (start 94.889589 102.3475) (end 95.91 102.3475) (width 0.25) (layer "B.Cu") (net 15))
 (segment (start 90.5 97.957911) (end 94.889589 102.3475) (width 0.25) (layer "B.Cu") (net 15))
 (segment (start 90.5 77) (end 90.5 97.957911) (width 0.25) (layer "B.Cu") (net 15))
 (segment (start 93 74.5) (end 90.5 77) (width 0.25) (layer "B.Cu") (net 15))
 (segment (start 93 73.4) (end 93 74.5) (width 0.25) (layer "B.Cu") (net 15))
 (segment (start 93 75) (end 93 73.35) (width 0.25) (layer "F.Cu") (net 17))
 (segment (start 90.5 98.5) (end 90.5 77.5) (width 0.25) (layer "F.Cu") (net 17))
 (segment (start 104.7825 100.5) (end 92.5 100.5) (width 0.25) (layer "F.Cu") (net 17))
 (segment (start 90.5 77.5) (end 93 75) (width 0.25) (layer "F.Cu") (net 17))
 (segment (start 92.5 100.5) (end 90.5 98.5) (width 0.25) (layer "F.Cu") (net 17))
 (segment (start 106.63 102.3475) (end 104.7825 100.5) (width 0.25) (layer "F.Cu") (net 17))
 (segment (start 93.37 102.3475) (end 90 98.9775) (width 0.25) (layer "B.Cu") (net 14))
 (segment (start 90 74.3) (end 91 73.3) (width 0.25) (layer "B.Cu") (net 14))
 (segment (start 90 98.9775) (end 90 74.3) (width 0.25) (layer "B.Cu") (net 14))
 (segment (start 91.5 101) (end 90 99.5) (width 0.25) (layer "F.Cu") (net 16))
 (segment (start 91 75.5) (end 91 73.35) (width 0.25) (layer "F.Cu") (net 16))
 (segment (start 90 99.5) (end 90 76.5) (width 0.25) (layer "F.Cu") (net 16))
 (segment (start 104.09 102.3475) (end 102.7425 101) (width 0.25) (layer "F.Cu") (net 16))
 (segment (start 102.7425 101) (end 91.5 101) (width 0.25) (layer "F.Cu") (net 16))
 (segment (start 90 76.5) (end 91 75.5) (width 0.25) (layer "F.Cu") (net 16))
 (segment (start 104.3 86.1) (end 104.3 80.588896) (width 0.25) (layer "B.Cu") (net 12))
 (segment (start 105.9 78.8) (end 107.2 77.5) (width 0.25) (layer "B.Cu") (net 12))
 (segment (start 103.175 95.477911) (end 105.552911 93.1) (width 0.25) (layer "B.Cu") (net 12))
 (segment (start 107.3 89.1) (end 104.3 86.1) (width 0.25) (layer "B.Cu") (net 12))
 (segment (start 103.175 95.7275) (end 103.175 95.477911) (width 0.25) (layer "B.Cu") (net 12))
 (segment (start 104.613803 80.275094) (end 105.9 78.988897) (width 0.25) (layer "B.Cu") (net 12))
 (segment (start 106.8 93.1) (end 107.3 92.6) (width 0.25) (layer "B.Cu") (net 12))
 (segment (start 105.9 78.988897) (end 105.9 78.8) (width 0.25) (layer "B.Cu") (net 12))
 (segment (start 105.552911 93.1) (end 106.8 93.1) (width 0.25) (layer "B.Cu") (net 12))
 (segment (start 107.2 77.5) (end 108.1 77.5) (width 0.25) (layer "B.Cu") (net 12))
 (segment (start 107.3 92.6) (end 107.3 89.1) (width 0.25) (layer "B.Cu") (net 12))
 (segment (start 104.3 80.588896) (end 104.613803 80.275094) (width 0.25) (layer "B.Cu") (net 12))
 (segment (start 107.6 89.761476) (end 107.6 92.5725) (width 0.25) (layer "F.Cu") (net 13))
 (segment (start 105.5245 81.5) (end 105.5245 87.685976) (width 0.25) (layer "F.Cu") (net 13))
 (segment (start 107.6 92.5725) (end 105.715 94.4575) (width 0.25) (layer "F.Cu") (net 13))
 (segment (start 105.5245 87.685976) (end 107.6 89.761476) (width 0.25) (layer "F.Cu") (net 13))
 (via (at 105.5245 81.5) (size 0.8) (drill 0.4) (layers "F.Cu" "B.Cu") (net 13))
 (segment (start 108.4 81.5) (end 105.5245 81.5) (width 0.25) (layer "B.Cu") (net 13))
 (segment (start 92.419511 95.532011) (end 95.109922 95.532011) (width 0.25) (layer "B.Cu") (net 18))
 (segment (start 92.125 95.2375) (end 92.419511 95.532011) (width 0.25) (layer "B.Cu") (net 18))
 (segment (start 106.8125 96.3) (end 107.875 95.2375) (width 0.25) (layer "B.Cu") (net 18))
 (segment (start 95.109922 95.532011) (end 96.432963 96.855052) (width 0.25) (layer "B.Cu") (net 18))
 (segment (start 104.910105 96.3) (end 106.8125 96.3) (width 0.25) (layer "B.Cu") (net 18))
 (segment (start 96.432963 96.855052) (end 104.355053 96.855052) (width 0.25) (layer "B.Cu") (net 18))
 (segment (start 104.355053 96.855052) (end 104.910105 96.3) (width 0.25) (layer "B.Cu") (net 18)))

